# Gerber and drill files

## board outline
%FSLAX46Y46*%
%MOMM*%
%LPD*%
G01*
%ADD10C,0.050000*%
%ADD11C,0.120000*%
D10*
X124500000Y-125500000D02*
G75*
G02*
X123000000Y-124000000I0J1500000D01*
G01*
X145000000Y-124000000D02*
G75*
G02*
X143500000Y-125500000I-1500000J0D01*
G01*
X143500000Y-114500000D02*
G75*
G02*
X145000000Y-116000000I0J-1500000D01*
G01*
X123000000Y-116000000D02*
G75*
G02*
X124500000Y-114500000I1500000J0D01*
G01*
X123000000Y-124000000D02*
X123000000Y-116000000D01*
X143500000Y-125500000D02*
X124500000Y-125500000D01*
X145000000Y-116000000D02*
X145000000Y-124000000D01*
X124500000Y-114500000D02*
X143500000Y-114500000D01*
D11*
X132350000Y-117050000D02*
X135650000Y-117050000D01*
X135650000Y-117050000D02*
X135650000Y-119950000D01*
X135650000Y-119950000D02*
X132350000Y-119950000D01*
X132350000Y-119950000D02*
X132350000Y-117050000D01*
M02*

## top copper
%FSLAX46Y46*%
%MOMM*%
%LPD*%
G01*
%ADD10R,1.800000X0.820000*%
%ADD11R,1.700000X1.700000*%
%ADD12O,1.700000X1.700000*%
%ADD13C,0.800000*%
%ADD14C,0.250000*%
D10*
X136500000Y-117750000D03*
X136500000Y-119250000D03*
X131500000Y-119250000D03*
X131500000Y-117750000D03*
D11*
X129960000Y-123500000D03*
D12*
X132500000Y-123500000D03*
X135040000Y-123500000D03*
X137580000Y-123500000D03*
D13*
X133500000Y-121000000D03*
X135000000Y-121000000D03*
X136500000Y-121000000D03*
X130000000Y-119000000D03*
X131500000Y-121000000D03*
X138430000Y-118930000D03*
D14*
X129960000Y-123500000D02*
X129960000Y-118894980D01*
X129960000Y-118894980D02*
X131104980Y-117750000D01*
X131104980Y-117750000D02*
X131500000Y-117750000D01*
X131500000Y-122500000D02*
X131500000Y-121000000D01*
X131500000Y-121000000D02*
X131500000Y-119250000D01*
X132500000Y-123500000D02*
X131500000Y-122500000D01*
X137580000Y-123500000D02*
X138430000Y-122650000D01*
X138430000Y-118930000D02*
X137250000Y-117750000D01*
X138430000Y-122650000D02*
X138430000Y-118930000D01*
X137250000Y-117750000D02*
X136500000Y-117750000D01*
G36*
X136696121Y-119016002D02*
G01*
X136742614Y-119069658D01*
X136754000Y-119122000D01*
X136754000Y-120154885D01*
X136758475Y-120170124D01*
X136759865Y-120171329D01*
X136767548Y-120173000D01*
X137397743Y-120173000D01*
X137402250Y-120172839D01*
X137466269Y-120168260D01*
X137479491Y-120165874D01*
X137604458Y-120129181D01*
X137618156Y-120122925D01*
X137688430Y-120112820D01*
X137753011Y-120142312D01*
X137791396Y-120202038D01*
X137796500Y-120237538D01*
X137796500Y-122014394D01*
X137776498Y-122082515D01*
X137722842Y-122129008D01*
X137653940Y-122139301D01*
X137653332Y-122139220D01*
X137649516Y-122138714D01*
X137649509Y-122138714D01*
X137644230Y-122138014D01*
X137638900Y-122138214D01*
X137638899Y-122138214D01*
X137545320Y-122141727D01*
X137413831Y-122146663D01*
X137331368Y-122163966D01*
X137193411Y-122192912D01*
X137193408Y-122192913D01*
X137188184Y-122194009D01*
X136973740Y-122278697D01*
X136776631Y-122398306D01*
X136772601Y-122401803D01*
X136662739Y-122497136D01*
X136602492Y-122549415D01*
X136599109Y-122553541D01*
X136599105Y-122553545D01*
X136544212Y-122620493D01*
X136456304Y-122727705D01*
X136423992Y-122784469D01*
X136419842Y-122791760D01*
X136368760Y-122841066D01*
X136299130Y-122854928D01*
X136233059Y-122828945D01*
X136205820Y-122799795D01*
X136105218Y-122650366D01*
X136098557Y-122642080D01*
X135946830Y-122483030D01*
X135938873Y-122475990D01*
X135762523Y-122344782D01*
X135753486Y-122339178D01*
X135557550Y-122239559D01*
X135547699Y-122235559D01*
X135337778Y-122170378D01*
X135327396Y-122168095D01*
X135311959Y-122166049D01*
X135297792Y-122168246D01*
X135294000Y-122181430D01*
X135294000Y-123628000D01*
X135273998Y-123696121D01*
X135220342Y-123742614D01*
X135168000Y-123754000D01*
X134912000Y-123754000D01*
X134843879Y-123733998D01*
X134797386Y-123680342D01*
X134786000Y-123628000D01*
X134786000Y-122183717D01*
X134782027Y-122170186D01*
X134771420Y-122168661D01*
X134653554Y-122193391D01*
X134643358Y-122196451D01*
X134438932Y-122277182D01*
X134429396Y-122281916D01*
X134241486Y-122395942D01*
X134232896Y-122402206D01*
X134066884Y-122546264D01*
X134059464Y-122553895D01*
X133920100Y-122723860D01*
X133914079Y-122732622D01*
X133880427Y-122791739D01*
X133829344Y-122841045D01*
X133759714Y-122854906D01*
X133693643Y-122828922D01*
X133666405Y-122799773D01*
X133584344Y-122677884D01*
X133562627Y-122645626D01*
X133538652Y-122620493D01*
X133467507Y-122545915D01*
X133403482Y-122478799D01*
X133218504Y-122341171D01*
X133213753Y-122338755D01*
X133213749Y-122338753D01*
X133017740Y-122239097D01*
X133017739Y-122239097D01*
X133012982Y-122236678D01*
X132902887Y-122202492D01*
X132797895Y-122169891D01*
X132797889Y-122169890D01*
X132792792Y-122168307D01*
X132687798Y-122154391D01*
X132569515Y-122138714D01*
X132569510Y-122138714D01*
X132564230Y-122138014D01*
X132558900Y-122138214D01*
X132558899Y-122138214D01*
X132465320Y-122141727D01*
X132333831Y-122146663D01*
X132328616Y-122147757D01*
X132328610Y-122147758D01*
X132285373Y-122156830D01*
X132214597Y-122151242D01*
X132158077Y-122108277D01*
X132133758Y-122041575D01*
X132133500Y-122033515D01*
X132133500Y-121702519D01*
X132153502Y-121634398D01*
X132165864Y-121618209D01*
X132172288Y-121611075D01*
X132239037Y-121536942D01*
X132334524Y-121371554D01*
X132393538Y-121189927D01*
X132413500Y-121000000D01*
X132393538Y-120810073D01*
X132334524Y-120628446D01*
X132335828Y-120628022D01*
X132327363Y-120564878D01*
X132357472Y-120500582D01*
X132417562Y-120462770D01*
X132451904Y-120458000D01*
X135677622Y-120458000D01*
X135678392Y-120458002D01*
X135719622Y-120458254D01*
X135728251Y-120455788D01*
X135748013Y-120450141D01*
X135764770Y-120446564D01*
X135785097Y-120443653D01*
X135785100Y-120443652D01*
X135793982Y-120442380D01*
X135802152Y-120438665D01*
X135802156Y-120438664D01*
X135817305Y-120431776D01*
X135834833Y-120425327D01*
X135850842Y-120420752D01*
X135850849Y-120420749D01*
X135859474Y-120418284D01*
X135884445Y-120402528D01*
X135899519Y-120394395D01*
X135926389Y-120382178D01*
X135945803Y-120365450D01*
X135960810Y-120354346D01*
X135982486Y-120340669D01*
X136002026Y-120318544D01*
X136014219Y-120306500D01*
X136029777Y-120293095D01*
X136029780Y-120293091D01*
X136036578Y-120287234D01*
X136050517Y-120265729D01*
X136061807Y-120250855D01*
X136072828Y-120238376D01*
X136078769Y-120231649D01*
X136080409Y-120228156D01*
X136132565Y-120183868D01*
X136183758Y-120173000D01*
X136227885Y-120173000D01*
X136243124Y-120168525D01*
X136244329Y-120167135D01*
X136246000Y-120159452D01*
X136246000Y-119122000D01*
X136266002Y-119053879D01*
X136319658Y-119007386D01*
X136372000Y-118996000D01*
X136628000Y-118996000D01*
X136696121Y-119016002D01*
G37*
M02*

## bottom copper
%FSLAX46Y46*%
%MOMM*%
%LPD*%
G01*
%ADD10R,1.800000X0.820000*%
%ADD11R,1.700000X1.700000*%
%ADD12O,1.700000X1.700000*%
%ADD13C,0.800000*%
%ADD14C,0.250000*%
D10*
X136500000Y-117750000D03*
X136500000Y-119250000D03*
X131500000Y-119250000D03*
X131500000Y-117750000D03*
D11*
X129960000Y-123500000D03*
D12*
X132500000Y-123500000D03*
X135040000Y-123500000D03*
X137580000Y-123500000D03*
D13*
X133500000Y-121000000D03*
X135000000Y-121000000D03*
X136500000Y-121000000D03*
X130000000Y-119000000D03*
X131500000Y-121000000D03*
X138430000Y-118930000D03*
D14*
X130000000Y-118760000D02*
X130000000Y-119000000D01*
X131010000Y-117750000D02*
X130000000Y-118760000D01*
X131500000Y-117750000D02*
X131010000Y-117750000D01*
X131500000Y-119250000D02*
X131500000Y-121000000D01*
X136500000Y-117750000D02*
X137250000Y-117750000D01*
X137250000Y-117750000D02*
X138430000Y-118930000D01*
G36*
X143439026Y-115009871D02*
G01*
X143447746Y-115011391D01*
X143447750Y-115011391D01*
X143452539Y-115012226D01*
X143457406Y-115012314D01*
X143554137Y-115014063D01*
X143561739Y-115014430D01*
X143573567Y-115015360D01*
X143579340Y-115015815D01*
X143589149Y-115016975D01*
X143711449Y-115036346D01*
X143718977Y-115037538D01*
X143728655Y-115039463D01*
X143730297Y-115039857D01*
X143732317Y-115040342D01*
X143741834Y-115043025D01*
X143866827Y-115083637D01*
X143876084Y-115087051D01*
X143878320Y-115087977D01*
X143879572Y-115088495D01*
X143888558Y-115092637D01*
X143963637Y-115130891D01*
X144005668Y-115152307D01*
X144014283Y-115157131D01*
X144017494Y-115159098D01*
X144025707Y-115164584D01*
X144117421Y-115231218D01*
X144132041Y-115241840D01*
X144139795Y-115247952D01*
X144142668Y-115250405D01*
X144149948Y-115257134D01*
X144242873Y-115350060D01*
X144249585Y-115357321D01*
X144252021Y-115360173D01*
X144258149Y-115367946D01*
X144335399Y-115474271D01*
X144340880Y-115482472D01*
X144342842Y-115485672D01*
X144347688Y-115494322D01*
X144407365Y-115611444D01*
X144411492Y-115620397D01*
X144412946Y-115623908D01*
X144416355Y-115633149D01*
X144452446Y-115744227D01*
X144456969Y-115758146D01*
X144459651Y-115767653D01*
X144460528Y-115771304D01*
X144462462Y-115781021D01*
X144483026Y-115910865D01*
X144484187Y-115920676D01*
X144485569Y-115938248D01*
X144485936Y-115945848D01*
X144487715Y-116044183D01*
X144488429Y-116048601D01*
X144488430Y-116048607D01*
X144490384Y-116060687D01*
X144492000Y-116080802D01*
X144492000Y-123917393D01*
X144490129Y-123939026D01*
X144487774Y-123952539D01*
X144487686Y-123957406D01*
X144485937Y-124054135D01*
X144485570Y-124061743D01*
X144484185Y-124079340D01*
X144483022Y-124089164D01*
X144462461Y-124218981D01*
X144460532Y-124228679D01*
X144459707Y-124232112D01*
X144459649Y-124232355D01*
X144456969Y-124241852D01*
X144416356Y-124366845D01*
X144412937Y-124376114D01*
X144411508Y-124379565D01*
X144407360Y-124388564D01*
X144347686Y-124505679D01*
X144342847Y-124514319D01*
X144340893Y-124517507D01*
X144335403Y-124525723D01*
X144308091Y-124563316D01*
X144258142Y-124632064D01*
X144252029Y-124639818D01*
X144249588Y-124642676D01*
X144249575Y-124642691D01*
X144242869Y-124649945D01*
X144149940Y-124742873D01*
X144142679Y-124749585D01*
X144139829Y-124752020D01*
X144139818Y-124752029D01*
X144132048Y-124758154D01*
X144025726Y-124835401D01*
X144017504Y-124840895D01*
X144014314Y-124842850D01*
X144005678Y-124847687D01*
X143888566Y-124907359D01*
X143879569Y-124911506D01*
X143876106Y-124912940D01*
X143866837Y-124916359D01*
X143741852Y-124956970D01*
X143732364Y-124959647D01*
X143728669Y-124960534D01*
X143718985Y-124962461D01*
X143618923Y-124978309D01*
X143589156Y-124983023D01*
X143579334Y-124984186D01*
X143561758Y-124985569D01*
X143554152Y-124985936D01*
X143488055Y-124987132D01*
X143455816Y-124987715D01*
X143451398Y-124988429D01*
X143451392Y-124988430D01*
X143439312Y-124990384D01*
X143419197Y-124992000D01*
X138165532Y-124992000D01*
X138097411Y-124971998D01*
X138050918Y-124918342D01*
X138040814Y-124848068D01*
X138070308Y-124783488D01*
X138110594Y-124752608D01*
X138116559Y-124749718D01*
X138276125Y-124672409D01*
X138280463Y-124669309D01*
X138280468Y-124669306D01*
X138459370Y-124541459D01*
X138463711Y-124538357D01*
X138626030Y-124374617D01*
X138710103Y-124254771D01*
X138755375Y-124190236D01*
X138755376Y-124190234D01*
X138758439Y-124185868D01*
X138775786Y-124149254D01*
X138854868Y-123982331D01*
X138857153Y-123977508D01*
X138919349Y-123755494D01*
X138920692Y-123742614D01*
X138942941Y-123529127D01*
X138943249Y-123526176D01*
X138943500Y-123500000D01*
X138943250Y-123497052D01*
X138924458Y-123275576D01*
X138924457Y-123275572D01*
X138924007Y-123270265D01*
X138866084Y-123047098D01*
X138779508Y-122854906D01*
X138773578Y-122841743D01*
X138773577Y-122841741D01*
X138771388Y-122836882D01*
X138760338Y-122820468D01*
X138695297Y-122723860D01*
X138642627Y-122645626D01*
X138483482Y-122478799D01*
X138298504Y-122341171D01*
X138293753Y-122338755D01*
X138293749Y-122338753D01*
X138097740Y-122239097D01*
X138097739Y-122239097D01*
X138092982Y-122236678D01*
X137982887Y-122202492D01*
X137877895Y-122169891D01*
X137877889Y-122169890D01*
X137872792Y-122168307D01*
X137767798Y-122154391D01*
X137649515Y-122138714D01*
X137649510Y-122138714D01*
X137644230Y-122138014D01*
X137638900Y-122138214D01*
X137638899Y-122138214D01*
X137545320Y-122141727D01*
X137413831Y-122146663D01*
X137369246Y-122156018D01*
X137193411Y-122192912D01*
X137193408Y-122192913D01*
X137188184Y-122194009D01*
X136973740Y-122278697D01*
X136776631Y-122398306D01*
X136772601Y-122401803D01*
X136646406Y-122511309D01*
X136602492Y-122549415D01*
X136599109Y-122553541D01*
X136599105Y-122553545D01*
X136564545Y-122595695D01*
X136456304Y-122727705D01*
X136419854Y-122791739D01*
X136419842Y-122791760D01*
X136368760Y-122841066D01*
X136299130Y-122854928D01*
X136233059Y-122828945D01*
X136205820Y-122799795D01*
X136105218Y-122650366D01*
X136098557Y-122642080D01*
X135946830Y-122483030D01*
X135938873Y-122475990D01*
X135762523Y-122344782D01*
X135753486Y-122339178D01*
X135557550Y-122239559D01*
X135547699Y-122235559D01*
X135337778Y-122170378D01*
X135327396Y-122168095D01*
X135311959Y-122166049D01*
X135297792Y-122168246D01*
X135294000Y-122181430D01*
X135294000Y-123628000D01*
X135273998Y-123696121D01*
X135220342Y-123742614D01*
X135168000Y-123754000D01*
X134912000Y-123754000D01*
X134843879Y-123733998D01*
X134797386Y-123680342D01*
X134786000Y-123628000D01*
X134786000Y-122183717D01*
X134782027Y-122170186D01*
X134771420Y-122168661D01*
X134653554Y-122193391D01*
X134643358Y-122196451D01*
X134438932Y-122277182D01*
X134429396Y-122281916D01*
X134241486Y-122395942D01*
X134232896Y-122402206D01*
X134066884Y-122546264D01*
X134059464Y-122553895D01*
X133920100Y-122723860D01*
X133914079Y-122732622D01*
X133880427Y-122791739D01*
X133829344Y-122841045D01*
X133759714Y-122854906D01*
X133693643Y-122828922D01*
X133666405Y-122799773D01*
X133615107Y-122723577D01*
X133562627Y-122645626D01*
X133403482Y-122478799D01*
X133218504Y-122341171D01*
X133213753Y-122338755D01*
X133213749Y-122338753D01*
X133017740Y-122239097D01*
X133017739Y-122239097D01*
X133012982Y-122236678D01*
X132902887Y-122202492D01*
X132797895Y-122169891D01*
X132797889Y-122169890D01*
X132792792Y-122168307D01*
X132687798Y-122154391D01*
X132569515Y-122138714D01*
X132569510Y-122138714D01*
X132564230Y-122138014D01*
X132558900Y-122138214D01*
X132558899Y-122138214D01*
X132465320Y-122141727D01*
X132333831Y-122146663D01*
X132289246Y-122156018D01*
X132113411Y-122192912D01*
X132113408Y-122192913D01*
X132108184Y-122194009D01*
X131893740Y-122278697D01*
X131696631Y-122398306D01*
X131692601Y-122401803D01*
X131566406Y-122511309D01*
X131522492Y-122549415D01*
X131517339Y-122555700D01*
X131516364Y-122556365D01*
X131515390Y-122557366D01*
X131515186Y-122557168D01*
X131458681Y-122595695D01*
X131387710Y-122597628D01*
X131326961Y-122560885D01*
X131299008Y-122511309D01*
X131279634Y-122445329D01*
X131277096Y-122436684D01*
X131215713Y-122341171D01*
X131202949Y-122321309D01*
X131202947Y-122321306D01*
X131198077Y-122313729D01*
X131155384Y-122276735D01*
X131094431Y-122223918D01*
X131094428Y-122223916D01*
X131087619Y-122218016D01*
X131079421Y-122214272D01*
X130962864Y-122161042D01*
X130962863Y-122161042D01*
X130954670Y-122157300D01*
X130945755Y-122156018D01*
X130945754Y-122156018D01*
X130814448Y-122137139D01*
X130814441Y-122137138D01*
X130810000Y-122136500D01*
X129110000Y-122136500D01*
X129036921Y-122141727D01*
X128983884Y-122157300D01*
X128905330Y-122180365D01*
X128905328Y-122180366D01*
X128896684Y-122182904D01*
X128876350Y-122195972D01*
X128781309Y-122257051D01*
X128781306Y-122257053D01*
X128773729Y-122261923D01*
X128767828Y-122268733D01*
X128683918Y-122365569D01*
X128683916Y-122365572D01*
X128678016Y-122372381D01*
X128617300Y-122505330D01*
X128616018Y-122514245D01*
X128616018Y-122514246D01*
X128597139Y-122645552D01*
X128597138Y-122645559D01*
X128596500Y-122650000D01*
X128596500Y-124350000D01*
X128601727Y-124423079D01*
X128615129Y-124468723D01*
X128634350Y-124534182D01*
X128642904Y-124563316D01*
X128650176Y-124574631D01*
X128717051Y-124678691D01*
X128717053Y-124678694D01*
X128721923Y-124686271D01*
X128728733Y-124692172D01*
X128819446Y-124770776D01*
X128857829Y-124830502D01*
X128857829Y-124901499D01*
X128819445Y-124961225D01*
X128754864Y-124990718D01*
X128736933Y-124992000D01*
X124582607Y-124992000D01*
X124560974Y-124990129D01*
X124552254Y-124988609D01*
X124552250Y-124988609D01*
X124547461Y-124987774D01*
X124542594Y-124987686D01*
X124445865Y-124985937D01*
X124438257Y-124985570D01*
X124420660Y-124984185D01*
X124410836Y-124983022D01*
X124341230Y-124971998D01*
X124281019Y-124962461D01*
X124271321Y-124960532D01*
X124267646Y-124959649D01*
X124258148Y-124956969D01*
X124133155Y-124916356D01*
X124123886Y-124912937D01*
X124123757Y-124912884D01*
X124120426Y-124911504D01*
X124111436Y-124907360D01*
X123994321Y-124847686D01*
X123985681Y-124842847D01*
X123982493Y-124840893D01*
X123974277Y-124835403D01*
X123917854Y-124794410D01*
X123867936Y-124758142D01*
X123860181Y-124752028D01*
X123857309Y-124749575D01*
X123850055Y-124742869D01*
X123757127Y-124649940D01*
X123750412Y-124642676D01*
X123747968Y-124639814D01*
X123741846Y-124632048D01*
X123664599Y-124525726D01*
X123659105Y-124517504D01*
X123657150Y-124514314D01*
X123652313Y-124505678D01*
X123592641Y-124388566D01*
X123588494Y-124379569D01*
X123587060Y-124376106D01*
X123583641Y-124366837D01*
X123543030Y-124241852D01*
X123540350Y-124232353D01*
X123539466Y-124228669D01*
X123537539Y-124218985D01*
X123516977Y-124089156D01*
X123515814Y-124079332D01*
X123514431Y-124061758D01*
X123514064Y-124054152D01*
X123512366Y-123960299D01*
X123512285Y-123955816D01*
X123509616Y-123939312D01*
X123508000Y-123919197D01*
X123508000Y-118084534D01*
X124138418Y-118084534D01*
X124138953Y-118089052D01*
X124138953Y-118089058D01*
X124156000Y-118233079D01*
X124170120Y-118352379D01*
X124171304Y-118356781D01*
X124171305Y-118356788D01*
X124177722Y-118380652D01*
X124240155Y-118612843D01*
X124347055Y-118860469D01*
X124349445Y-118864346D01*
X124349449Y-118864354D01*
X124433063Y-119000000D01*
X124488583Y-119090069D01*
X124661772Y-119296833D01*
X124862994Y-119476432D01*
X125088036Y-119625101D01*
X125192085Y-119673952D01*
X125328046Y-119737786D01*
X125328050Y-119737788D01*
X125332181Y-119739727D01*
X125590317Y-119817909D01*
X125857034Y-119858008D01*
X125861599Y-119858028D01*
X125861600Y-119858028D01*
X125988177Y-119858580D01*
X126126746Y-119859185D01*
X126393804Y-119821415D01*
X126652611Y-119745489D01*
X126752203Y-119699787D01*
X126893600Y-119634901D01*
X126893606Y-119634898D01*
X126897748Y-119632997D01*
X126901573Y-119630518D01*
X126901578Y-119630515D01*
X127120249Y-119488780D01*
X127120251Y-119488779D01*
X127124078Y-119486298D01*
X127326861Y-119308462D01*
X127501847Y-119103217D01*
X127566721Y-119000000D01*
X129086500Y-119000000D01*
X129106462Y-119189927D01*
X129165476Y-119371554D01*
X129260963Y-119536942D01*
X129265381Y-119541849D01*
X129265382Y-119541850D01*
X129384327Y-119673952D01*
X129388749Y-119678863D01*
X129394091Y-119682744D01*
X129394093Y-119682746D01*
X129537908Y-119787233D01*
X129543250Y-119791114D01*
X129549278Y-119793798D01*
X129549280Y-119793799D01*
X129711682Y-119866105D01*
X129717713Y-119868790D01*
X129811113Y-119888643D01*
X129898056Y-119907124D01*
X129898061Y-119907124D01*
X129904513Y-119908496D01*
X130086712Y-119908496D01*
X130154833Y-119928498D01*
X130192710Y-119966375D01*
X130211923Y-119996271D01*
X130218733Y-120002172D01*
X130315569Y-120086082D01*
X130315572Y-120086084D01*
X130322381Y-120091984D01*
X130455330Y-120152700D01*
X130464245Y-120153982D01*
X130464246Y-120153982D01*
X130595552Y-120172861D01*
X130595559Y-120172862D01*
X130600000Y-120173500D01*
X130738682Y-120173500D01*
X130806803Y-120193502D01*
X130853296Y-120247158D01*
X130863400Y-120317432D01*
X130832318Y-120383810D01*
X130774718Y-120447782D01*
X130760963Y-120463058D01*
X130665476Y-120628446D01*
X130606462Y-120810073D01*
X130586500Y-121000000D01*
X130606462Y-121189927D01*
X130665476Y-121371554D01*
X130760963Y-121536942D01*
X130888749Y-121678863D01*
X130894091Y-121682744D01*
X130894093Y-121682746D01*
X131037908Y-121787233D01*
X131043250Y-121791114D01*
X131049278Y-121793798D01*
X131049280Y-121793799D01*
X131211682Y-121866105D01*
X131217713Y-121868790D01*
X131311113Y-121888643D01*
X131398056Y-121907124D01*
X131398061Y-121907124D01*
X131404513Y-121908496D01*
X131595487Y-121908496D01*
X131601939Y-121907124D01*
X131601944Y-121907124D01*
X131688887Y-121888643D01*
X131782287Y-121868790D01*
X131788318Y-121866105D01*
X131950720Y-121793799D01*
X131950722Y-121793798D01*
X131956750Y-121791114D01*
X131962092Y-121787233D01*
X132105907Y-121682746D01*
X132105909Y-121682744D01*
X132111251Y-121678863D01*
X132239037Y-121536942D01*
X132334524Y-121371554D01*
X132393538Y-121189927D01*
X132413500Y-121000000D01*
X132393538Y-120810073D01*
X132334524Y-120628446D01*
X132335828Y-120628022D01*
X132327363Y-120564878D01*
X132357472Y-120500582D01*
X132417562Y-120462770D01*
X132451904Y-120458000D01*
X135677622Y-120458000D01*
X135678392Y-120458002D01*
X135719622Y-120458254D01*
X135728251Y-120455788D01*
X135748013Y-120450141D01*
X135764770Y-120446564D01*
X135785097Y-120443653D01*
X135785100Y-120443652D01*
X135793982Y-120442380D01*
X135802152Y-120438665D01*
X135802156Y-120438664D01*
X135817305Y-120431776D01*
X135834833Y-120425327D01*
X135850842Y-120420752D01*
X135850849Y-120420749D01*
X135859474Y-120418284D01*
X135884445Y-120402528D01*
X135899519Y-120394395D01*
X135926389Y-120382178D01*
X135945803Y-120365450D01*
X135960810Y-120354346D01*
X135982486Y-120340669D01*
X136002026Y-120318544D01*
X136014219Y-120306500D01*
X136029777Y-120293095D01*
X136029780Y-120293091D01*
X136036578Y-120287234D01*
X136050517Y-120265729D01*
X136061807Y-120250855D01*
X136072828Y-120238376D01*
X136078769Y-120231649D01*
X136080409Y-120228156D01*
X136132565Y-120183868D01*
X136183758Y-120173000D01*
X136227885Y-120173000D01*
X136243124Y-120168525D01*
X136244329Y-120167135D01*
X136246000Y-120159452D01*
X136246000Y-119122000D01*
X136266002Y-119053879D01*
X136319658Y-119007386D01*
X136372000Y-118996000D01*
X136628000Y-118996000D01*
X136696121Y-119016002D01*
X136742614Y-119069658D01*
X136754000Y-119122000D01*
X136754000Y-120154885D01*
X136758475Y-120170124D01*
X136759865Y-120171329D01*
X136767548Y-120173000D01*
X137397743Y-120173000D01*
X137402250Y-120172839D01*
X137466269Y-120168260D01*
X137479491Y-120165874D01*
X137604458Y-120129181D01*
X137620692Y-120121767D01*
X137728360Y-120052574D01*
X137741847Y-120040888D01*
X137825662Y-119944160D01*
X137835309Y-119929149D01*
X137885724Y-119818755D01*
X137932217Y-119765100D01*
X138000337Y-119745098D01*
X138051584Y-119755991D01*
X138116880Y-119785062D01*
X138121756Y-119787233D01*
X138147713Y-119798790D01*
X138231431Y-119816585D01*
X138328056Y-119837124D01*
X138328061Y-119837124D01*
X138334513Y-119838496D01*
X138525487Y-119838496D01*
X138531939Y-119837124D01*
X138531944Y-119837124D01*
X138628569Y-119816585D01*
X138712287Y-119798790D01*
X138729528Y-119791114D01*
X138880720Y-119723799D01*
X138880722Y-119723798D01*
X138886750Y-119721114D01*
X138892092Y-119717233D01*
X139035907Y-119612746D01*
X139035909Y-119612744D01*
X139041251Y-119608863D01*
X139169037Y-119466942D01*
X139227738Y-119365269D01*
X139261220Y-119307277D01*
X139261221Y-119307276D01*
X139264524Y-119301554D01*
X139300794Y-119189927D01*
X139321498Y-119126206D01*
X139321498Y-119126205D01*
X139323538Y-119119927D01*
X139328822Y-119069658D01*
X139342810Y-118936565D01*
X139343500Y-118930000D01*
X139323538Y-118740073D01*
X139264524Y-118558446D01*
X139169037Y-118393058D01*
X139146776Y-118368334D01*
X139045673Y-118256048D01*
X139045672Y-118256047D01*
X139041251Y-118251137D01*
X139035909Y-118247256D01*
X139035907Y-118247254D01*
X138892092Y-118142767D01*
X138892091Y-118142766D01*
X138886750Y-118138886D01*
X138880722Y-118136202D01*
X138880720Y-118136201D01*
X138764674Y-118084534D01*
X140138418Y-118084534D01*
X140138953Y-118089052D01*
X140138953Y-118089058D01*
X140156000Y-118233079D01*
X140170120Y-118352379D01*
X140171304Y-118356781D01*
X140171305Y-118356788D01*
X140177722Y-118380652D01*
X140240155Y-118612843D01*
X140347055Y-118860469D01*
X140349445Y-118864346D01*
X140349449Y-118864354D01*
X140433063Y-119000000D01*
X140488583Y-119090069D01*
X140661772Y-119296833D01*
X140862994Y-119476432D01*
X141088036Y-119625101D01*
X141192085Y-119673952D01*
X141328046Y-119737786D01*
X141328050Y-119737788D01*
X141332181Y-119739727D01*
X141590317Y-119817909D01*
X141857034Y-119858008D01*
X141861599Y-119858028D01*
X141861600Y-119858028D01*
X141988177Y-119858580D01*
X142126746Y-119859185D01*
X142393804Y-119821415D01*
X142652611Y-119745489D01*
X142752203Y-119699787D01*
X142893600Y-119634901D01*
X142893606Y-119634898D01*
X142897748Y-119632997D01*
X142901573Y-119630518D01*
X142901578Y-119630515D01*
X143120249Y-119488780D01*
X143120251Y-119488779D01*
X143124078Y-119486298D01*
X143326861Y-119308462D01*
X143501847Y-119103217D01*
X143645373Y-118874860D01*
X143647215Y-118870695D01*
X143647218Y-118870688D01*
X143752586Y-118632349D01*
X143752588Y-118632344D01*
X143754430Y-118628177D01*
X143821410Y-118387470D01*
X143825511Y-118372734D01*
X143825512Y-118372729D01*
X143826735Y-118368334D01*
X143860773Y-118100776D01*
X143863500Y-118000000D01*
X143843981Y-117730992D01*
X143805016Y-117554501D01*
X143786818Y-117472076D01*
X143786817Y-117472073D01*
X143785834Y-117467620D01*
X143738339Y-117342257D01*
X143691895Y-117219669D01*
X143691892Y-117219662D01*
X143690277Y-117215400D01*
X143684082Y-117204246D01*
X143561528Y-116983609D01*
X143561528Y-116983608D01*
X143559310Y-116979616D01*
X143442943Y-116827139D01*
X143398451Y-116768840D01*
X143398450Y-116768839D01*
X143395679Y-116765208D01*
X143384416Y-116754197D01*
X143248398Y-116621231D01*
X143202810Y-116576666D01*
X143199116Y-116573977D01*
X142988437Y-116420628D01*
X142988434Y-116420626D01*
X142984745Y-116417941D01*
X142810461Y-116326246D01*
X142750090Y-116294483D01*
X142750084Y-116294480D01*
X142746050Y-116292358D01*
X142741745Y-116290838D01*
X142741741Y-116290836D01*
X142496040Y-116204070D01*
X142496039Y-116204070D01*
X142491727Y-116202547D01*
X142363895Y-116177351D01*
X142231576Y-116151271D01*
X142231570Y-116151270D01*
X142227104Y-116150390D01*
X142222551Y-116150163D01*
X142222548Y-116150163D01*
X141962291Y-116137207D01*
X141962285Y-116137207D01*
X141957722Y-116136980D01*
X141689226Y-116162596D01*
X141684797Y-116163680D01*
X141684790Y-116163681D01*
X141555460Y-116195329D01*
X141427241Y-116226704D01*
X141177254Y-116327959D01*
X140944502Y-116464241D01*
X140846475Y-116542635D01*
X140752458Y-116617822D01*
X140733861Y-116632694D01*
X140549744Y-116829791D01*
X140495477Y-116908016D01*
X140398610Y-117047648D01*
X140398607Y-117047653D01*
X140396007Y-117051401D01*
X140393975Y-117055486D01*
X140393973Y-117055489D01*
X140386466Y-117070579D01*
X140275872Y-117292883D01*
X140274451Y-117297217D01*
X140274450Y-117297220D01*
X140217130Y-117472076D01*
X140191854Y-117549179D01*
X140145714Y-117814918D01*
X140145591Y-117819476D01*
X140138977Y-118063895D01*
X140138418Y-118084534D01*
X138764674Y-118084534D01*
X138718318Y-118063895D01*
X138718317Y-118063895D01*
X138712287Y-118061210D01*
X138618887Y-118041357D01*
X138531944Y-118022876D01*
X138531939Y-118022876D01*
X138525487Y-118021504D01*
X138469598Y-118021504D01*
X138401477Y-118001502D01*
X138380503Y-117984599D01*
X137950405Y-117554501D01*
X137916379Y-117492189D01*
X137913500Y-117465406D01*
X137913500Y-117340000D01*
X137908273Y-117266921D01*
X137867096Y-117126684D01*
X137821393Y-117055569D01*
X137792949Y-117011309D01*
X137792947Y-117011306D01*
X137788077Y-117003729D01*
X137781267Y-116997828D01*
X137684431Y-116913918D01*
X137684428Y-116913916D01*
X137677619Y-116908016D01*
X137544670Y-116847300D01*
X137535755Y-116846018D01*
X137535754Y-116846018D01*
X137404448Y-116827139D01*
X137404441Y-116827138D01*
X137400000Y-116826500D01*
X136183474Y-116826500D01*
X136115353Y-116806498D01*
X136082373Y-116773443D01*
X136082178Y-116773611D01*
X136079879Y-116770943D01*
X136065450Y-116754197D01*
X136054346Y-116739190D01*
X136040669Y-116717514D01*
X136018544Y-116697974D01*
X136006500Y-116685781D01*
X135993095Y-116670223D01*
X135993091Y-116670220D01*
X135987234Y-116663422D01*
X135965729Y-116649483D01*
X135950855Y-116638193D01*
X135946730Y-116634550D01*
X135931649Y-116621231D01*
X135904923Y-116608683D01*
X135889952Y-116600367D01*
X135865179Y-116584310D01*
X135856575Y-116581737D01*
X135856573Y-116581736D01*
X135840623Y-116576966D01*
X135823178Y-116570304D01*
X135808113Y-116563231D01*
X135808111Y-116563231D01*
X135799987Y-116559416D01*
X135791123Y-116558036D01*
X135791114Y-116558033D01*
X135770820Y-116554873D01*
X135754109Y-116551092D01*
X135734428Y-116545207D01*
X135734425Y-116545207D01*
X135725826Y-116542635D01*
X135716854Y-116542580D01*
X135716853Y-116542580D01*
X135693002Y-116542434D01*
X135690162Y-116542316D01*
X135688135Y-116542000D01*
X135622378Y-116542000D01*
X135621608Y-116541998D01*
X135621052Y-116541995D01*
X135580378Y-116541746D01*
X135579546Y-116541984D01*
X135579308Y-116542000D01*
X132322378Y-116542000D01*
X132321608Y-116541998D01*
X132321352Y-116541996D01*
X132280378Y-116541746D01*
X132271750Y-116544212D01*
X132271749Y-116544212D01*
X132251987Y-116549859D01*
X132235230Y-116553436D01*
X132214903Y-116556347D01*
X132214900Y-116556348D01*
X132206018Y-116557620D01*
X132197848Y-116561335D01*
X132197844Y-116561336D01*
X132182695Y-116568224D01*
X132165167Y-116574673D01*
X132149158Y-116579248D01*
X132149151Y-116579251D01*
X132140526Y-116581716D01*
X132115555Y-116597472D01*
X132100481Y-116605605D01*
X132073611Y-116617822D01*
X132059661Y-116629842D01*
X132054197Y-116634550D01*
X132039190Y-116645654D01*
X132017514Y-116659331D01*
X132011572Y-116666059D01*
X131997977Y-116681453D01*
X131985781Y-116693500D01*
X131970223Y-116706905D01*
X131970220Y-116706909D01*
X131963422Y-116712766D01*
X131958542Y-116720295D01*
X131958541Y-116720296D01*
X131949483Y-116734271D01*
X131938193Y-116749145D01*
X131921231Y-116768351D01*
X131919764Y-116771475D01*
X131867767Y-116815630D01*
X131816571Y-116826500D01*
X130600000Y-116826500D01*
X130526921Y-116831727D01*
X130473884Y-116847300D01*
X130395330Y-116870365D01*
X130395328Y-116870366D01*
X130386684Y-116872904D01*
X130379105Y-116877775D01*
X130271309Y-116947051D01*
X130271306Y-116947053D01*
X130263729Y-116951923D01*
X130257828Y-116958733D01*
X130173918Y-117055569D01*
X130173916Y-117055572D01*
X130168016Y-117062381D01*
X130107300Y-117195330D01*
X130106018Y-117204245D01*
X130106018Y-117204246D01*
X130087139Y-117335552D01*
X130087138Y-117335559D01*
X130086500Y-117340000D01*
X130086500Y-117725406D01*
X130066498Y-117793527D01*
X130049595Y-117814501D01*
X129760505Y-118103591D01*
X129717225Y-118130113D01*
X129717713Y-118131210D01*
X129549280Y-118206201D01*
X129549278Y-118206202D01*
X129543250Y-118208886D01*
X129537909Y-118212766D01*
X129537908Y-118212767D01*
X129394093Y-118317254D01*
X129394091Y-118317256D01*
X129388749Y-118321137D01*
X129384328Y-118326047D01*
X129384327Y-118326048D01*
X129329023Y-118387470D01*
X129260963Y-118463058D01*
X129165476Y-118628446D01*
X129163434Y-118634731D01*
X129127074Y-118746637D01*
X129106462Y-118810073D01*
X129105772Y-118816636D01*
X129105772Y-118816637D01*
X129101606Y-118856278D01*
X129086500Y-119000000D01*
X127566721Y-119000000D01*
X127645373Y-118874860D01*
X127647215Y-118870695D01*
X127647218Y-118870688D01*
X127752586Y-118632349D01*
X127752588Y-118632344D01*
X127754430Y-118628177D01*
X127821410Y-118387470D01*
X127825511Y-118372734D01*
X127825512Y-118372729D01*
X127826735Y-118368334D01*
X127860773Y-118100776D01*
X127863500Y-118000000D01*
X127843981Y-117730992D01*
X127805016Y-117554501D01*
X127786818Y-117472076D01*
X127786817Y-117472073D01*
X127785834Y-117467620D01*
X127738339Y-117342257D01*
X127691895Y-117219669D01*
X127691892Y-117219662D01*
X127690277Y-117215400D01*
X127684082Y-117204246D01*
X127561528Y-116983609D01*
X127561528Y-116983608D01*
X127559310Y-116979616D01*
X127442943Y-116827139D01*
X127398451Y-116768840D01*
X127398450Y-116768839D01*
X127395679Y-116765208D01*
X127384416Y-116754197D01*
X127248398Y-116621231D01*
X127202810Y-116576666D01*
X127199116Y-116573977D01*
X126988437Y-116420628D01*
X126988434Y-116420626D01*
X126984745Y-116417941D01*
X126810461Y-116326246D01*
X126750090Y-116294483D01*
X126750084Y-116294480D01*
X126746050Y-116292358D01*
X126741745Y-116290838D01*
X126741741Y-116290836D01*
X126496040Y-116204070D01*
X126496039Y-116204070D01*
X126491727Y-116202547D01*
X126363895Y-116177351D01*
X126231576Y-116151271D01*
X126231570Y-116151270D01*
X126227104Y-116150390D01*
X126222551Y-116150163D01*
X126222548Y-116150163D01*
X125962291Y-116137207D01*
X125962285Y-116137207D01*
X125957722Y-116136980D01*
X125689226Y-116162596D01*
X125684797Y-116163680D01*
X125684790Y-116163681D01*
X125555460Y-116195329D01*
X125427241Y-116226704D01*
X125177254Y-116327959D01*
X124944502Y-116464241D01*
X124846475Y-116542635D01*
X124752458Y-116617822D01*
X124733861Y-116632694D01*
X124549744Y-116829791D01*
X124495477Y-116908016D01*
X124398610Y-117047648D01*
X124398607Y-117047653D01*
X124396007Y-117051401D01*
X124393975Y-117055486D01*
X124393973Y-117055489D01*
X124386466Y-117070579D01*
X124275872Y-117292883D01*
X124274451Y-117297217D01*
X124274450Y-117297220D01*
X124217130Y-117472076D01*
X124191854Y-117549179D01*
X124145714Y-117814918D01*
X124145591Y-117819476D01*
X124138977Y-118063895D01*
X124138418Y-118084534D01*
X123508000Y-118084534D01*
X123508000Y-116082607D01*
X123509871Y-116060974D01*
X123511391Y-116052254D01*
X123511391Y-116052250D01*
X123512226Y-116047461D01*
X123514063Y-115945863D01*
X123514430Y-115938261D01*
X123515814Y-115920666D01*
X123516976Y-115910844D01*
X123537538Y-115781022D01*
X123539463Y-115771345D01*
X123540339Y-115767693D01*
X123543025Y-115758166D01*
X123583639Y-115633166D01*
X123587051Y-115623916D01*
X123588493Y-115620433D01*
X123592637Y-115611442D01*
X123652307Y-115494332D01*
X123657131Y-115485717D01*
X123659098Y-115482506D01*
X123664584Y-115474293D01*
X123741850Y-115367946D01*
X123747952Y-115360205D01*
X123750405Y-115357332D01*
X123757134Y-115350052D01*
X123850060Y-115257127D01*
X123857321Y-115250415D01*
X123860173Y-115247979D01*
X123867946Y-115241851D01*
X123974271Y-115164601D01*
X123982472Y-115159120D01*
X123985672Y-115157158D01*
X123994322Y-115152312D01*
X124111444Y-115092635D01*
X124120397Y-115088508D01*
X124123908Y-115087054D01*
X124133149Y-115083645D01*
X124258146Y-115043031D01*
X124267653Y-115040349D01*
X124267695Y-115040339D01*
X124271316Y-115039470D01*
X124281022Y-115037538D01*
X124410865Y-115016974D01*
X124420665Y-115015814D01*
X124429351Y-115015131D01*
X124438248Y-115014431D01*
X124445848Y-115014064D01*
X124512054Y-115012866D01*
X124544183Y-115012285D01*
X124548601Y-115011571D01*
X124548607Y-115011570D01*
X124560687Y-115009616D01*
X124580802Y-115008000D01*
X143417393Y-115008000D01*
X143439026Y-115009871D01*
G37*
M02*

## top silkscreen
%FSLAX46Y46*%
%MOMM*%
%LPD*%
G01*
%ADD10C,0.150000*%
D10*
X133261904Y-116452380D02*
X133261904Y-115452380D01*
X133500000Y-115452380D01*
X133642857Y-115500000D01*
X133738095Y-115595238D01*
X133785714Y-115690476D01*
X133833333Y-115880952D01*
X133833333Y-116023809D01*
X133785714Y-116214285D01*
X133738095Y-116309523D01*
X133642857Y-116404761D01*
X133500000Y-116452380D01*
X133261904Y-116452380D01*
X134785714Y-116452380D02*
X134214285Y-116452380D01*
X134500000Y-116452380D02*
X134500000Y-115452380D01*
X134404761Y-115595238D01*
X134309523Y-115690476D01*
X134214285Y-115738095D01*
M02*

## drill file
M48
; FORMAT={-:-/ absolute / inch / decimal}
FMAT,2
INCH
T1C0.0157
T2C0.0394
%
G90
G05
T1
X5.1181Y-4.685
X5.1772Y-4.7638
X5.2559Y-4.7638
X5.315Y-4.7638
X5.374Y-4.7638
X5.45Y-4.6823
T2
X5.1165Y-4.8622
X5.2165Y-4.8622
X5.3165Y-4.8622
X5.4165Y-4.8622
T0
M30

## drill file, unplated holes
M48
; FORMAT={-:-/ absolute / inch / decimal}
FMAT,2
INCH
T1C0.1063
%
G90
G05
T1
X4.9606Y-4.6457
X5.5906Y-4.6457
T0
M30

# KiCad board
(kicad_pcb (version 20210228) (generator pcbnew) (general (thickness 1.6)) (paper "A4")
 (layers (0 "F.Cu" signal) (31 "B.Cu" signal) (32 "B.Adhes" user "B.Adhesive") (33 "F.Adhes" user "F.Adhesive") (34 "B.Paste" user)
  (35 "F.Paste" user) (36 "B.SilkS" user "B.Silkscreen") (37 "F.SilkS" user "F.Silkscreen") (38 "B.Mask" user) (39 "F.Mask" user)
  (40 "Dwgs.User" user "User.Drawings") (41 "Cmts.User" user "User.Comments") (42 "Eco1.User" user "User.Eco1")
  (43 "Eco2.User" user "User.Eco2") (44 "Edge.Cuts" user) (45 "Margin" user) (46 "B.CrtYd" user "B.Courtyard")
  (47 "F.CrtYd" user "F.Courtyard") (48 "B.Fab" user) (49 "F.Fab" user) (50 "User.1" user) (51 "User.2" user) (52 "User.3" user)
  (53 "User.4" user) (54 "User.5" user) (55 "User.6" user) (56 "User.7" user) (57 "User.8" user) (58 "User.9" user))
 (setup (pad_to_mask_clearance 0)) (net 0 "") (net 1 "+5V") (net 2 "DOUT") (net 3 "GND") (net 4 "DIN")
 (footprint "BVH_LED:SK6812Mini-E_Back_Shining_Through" (layer "F.Cu") (at 134 118.5)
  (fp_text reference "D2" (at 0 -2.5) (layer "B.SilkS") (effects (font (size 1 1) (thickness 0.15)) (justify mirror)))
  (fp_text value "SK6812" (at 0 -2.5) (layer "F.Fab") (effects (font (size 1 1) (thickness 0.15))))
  (pad "1" smd rect (at -2.5 -0.75) (size 1.8 0.82) (layers "B.Cu" "B.Paste" "B.Mask") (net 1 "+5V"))
  (pad "2" smd rect (at -2.5 0.75) (size 1.8 0.82) (layers "B.Cu" "B.Paste" "B.Mask") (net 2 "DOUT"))
  (pad "3" smd rect (at 2.5 0.75) (size 1.8 0.82) (layers "B.Cu" "B.Paste" "B.Mask") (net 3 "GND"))
  (pad "4" smd rect (at 2.5 -0.75) (size 1.8 0.82) (layers "B.Cu" "B.Paste" "B.Mask") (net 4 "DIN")))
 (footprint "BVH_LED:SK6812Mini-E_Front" (layer "F.Cu") (at 134 118.5)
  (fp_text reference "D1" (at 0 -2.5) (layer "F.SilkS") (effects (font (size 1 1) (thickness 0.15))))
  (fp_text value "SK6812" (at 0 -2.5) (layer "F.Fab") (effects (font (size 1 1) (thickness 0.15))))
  (fp_rect (start -1.65 -1.45) (end 1.65 1.45) (layer "Edge.Cuts") (width 0.12) (fill none))
  (pad "1" smd rect (at -2.5 -0.75) (locked) (size 1.8 0.82) (layers "F.Cu" "F.Paste" "F.Mask") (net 1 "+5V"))
  (pad "2" smd rect (at -2.5 0.75) (locked) (size 1.8 0.82) (layers "F.Cu" "F.Paste" "F.Mask") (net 2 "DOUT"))
  (pad "3" smd rect (at 2.5 0.75) (locked) (size 1.8 0.82) (layers "F.Cu" "F.Paste" "F.Mask") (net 3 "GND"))
  (pad "4" smd rect (at 2.5 -0.75) (locked) (size 1.8 0.82) (layers "F.Cu" "F.Paste" "F.Mask") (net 4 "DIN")))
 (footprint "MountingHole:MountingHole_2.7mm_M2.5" (layer "F.Cu") (at 126 118)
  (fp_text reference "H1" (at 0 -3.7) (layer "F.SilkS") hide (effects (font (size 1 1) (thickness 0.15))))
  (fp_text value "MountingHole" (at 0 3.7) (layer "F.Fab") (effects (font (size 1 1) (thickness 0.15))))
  (pad "1" np_thru_hole circle (at 0 0) (locked) (size 2.7 2.7) (drill 2.7) (layers *.Cu *.Mask)))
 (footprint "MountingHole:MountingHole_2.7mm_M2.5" (layer "F.Cu") (at 142 118)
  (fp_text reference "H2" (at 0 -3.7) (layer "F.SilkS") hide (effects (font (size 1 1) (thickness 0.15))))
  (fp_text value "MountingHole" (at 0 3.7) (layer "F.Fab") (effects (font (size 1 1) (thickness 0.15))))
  (pad "1" np_thru_hole circle (at 0 0) (locked) (size 2.7 2.7) (drill 2.7) (layers *.Cu *.Mask)))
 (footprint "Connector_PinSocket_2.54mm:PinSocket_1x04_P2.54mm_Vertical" (layer "B.Cu") (at 129.96 123.5 -90)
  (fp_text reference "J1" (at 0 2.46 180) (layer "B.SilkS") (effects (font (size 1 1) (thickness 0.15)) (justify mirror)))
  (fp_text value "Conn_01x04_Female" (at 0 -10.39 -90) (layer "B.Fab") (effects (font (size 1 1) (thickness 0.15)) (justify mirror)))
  (pad "1" thru_hole rect (at 0 0 270) (locked) (size 1.7 1.7) (drill 1) (layers *.Cu *.Mask) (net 1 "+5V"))
  (pad "2" thru_hole oval (at 0 -2.54 270) (locked) (size 1.7 1.7) (drill 1) (layers *.Cu *.Mask) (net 2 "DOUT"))
  (pad "3" thru_hole oval (at 0 -5.08 270) (locked) (size 1.7 1.7) (drill 1) (layers *.Cu *.Mask) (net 3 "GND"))
  (pad "4" thru_hole oval (at 0 -7.62 270) (locked) (size 1.7 1.7) (drill 1) (layers *.Cu *.Mask) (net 4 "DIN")))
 (gr_arc (start 124.5 116) (end 124.5 114.5) (angle -90) (layer "Edge.Cuts") (width 0.05))
 (gr_line (start 124.5 114.5) (end 143.5 114.5) (layer "Edge.Cuts") (width 0.05))
 (gr_line (start 143.5 125.5) (end 124.5 125.5) (layer "Edge.Cuts") (width 0.05))
 (gr_arc (start 124.5 124) (end 123 124) (angle -90) (layer "Edge.Cuts") (width 0.05))
 (gr_line (start 145 116) (end 145 124) (layer "Edge.Cuts") (width 0.05))
 (gr_arc (start 143.5 124) (end 143.5 125.5) (angle -90) (layer "Edge.Cuts") (width 0.05))
 (gr_arc (start 143.5 116) (end 145 116) (angle -90) (layer "Edge.Cuts") (width 0.05))
 (gr_line (start 123 124) (end 123 116) (layer "Edge.Cuts") (width 0.05))
 (segment (start 131.5 121) (end 131.5 119.25) (width 0.25) (layer "F.Cu") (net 2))
 (segment (start 131.5 122.5) (end 131.5 121) (width 0.25) (layer "F.Cu") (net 2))
 (segment (start 132.5 123.5) (end 131.5 122.5) (width 0.25) (layer "F.Cu") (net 2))
 (via (at 131.5 121) (size 0.8) (drill 0.4) (layers "F.Cu" "B.Cu") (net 2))
 (segment (start 131.5 119.25) (end 131.5 121) (width 0.25) (layer "B.Cu") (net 2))
 (via (at 135 121) (size 0.8) (drill 0.4) (layers "F.Cu" "B.Cu") (free) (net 3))
 (via (at 136.5 121) (size 0.8) (drill 0.4) (layers "F.Cu" "B.Cu") (free) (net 3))
 (via (at 133.5 121) (size 0.8) (drill 0.4) (layers "F.Cu" "B.Cu") (free) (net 3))
 (segment (start 129.96 118.89498) (end 131.10498 117.75) (width 0.25) (layer "F.Cu") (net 1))
 (segment (start 129.96 123.5) (end 129.96 118.89498) (width 0.25) (layer "F.Cu") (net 1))
 (segment (start 131.10498 117.75) (end 131.5 117.75) (width 0.25) (layer "F.Cu") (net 1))
 (via (at 130 119) (size 0.8) (drill 0.4) (layers "F.Cu" "B.Cu") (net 1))
 (segment (start 130 118.76) (end 130 119) (width 0.25) (layer "B.Cu") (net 1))
 (segment (start 131.01 117.75) (end 130 118.76) (width 0.25) (layer "B.Cu") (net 1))
 (segment (start 131.5 117.75) (end 131.01 117.75) (width 0.25) (layer "B.Cu") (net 1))
 (segment (start 137.58 123.5) (end 138.43 122.65) (width 0.25) (layer "F.Cu") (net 4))
 (segment (start 137.25 117.75) (end 136.5 117.75) (width 0.25) (layer "F.Cu") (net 4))
 (segment (start 138.43 118.93) (end 137.25 117.75) (width 0.25) (layer "F.Cu") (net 4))
 (segment (start 138.43 122.65) (end 138.43 118.93) (width 0.25) (layer "F.Cu") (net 4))
 (via (at 138.43 118.93) (size 0.8) (drill 0.4) (layers "F.Cu" "B.Cu") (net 4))
 (segment (start 137.25 117.75) (end 138.43 118.93) (width 0.25) (layer "B.Cu") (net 4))
 (segment (start 136.5 117.75) (end 137.25 117.75) (width 0.25) (layer "B.Cu") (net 4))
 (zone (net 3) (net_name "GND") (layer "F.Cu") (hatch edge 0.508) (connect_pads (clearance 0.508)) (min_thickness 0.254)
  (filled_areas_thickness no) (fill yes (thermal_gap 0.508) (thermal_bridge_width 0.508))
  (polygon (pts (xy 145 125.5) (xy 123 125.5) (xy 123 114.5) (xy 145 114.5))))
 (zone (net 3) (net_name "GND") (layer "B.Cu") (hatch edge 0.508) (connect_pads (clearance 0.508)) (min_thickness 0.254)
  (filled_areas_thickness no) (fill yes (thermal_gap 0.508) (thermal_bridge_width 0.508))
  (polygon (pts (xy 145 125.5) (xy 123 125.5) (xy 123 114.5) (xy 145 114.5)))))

